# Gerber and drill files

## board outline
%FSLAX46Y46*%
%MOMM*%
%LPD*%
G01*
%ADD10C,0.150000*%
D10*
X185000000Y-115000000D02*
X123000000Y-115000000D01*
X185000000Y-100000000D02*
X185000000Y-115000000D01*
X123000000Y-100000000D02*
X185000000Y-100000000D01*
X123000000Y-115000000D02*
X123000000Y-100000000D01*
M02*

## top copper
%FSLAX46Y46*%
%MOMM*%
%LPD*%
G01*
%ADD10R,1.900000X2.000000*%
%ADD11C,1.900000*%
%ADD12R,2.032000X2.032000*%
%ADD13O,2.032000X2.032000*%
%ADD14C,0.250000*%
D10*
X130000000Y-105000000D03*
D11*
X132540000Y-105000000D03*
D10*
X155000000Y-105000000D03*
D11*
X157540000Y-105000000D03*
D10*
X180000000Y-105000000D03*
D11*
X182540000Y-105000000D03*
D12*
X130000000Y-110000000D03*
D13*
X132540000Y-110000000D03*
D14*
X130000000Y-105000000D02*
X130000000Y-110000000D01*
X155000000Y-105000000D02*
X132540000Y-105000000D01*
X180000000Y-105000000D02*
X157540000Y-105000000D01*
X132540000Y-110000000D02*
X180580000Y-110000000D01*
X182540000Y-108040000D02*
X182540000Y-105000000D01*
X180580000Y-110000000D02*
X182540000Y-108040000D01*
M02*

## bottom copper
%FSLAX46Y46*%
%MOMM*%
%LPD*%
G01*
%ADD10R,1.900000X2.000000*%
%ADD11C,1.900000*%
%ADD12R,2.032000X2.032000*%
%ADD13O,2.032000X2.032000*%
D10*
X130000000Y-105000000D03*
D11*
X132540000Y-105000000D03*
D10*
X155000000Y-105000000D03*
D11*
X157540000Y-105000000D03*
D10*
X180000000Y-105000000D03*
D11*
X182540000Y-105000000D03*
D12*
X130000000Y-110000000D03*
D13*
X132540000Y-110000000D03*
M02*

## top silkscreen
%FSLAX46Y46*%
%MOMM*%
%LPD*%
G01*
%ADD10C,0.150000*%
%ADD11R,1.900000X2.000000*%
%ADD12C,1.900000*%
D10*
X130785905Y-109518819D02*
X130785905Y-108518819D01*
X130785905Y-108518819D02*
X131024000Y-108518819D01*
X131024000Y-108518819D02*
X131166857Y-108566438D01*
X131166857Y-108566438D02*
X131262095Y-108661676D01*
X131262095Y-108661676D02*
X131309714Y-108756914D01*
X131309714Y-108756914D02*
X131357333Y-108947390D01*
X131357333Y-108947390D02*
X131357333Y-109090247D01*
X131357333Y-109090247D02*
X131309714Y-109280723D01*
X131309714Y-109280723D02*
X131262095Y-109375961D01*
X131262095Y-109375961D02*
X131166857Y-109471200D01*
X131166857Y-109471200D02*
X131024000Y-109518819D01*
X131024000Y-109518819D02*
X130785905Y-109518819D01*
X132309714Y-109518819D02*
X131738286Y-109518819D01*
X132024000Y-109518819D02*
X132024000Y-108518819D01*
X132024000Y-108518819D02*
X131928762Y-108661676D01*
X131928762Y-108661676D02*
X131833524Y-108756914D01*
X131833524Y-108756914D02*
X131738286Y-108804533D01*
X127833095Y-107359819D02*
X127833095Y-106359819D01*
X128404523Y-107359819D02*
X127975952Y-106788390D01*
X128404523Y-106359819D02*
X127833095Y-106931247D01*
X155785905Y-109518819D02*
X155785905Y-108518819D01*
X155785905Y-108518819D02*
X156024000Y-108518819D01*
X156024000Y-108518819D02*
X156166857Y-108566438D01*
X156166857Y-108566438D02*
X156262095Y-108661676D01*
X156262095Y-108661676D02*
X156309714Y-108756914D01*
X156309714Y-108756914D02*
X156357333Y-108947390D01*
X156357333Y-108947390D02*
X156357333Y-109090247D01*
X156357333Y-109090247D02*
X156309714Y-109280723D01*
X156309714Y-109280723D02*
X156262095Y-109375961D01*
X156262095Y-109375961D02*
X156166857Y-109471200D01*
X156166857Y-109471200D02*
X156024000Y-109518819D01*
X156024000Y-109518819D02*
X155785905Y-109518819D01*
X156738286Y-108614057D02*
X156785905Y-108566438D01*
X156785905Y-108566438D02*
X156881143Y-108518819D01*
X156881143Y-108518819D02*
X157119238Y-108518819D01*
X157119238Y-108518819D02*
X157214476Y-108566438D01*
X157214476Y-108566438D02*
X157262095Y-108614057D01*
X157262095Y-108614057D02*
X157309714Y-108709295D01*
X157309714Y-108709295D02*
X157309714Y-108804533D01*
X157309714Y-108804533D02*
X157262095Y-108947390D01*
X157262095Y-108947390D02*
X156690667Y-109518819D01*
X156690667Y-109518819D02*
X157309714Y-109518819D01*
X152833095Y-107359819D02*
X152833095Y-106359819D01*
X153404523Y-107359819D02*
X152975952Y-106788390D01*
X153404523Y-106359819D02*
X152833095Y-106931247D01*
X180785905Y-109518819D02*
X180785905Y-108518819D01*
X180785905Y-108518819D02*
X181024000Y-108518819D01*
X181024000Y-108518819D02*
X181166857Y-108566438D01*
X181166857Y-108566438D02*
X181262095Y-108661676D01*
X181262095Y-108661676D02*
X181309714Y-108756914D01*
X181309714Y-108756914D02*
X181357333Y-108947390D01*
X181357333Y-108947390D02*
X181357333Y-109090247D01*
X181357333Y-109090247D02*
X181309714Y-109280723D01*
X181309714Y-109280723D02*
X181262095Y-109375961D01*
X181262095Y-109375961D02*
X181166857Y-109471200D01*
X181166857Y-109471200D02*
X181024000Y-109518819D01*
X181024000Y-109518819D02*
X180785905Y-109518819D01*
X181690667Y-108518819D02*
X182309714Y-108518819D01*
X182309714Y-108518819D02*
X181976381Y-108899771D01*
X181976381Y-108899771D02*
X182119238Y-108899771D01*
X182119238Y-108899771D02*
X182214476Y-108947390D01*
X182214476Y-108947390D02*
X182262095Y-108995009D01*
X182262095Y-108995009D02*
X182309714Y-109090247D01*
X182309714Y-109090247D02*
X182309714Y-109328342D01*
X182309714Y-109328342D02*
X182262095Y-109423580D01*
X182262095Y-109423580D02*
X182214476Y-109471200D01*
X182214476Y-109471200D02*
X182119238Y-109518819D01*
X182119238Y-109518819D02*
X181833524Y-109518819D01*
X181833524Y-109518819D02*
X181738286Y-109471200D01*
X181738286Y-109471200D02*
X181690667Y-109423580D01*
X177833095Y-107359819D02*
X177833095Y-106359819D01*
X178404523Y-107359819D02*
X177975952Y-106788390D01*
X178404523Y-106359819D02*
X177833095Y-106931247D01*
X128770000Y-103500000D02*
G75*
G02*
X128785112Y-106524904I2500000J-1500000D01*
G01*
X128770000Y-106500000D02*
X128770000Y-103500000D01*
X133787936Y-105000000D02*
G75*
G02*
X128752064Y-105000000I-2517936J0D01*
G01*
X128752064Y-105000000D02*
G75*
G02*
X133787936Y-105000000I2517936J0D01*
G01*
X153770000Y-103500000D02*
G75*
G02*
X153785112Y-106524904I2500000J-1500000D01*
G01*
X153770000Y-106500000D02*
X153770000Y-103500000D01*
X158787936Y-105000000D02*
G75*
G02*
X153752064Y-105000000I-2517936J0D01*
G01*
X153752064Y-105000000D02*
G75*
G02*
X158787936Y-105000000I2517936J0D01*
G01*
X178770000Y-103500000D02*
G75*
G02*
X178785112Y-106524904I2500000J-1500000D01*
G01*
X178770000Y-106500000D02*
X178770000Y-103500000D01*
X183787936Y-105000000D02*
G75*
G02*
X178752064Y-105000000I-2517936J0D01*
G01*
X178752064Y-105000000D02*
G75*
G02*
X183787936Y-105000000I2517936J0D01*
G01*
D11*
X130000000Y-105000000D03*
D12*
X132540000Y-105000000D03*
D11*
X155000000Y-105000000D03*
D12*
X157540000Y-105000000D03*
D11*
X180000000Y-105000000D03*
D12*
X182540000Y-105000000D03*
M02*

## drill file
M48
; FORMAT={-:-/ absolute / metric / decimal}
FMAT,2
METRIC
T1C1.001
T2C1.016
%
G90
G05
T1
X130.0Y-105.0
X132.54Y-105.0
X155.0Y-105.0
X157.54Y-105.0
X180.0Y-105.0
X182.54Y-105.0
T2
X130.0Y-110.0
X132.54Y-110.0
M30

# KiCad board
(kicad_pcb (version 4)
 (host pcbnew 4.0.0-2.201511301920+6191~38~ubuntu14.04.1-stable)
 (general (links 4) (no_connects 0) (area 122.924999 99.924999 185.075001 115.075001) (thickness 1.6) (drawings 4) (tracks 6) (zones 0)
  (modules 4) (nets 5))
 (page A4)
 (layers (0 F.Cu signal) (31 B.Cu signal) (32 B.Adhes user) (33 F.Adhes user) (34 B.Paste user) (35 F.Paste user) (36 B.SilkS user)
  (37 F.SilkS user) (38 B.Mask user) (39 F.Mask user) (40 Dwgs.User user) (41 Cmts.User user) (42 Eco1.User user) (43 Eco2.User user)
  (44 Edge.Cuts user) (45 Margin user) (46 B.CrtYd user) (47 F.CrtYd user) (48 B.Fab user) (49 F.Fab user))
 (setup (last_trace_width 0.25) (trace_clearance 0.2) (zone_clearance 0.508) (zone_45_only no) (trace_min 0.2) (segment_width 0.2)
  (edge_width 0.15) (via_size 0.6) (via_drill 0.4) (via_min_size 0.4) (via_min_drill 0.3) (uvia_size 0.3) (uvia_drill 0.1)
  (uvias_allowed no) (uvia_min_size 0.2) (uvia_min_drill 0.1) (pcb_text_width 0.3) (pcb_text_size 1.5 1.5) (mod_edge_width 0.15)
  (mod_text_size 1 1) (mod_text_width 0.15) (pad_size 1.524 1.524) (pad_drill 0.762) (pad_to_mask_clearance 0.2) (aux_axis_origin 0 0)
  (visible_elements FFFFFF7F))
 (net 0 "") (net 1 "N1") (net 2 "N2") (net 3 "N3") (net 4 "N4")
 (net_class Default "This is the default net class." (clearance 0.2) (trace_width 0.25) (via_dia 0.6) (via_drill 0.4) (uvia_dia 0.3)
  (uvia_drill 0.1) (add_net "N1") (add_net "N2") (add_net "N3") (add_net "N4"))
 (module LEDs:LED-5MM (layer F.Cu) (at 130 105)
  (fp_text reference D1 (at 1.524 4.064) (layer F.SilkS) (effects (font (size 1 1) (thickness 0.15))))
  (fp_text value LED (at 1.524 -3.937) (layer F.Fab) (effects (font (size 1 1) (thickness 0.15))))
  (fp_arc (start 1.27 0) (end -1.23 -1.5) (angle 297.5) (layer F.SilkS) (width 0.15))
  (fp_line (start -1.23 1.5) (end -1.23 -1.5) (layer F.SilkS) (width 0.15))
  (fp_circle (center 1.27 0) (end 0.97 -2.5) (layer F.SilkS) (width 0.15))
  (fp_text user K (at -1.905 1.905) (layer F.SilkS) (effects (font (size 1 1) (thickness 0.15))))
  (pad 1 thru_hole rect (at 0 0 90) (size 2 1.9) (drill 1.00076) (layers *.Cu *.Mask F.SilkS) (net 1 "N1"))
  (pad 2 thru_hole circle (at 2.54 0) (size 1.9 1.9) (drill 1.00076) (layers *.Cu *.Mask F.SilkS) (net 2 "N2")))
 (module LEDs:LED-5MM (layer F.Cu) (at 155 105)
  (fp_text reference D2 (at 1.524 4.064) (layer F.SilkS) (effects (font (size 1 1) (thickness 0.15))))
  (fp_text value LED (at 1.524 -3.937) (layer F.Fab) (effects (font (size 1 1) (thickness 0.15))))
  (fp_arc (start 1.27 0) (end -1.23 -1.5) (angle 297.5) (layer F.SilkS) (width 0.15))
  (fp_line (start -1.23 1.5) (end -1.23 -1.5) (layer F.SilkS) (width 0.15))
  (fp_circle (center 1.27 0) (end 0.97 -2.5) (layer F.SilkS) (width 0.15))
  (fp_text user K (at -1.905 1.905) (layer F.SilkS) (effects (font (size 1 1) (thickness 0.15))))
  (pad 1 thru_hole rect (at 0 0 90) (size 2 1.9) (drill 1.00076) (layers *.Cu *.Mask F.SilkS) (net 2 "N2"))
  (pad 2 thru_hole circle (at 2.54 0) (size 1.9 1.9) (drill 1.00076) (layers *.Cu *.Mask F.SilkS) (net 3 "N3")))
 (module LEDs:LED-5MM (layer F.Cu) (at 180 105)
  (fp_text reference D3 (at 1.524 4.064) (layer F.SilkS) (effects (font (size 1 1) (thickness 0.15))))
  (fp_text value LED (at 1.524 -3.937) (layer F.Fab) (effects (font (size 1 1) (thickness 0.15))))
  (fp_arc (start 1.27 0) (end -1.23 -1.5) (angle 297.5) (layer F.SilkS) (width 0.15))
  (fp_line (start -1.23 1.5) (end -1.23 -1.5) (layer F.SilkS) (width 0.15))
  (fp_circle (center 1.27 0) (end 0.97 -2.5) (layer F.SilkS) (width 0.15))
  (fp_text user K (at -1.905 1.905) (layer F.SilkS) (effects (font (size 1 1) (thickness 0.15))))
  (pad 1 thru_hole rect (at 0 0 90) (size 2 1.9) (drill 1.00076) (layers *.Cu *.Mask F.SilkS) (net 3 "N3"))
  (pad 2 thru_hole circle (at 2.54 0) (size 1.9 1.9) (drill 1.00076) (layers *.Cu *.Mask F.SilkS) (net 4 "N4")))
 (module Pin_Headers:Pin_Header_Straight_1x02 (layer B.Cu) (at 130 110 270)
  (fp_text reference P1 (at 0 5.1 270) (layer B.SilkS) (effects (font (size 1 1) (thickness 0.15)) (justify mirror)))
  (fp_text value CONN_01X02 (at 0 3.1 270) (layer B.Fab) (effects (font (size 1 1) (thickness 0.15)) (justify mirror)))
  (pad 1 thru_hole rect (at 0 0 270) (size 2.032 2.032) (drill 1.016) (layers *.Cu *.Mask B.SilkS) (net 1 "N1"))
  (pad 2 thru_hole oval (at 0 -2.54 270) (size 2.032 2.032) (drill 1.016) (layers *.Cu *.Mask B.SilkS) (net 4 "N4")))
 (gr_line (start 185 115) (end 123 115) (angle 90) (layer Edge.Cuts) (width 0.15))
 (gr_line (start 185 100) (end 185 115) (angle 90) (layer Edge.Cuts) (width 0.15))
 (gr_line (start 123 100) (end 185 100) (angle 90) (layer Edge.Cuts) (width 0.15))
 (gr_line (start 123 115) (end 123 100) (angle 90) (layer Edge.Cuts) (width 0.15))
 (segment (start 130 105) (end 130 110) (width 0.25) (layer F.Cu) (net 1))
 (segment (start 155 105) (end 132.54 105) (width 0.25) (layer F.Cu) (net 2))
 (segment (start 180 105) (end 157.54 105) (width 0.25) (layer F.Cu) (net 3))
 (segment (start 132.54 110) (end 180.58 110) (width 0.25) (layer F.Cu) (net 4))
 (segment (start 182.54 108.04) (end 182.54 105) (width 0.25) (layer F.Cu) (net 4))
 (segment (start 180.58 110) (end 182.54 108.04) (width 0.25) (layer F.Cu) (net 4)))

